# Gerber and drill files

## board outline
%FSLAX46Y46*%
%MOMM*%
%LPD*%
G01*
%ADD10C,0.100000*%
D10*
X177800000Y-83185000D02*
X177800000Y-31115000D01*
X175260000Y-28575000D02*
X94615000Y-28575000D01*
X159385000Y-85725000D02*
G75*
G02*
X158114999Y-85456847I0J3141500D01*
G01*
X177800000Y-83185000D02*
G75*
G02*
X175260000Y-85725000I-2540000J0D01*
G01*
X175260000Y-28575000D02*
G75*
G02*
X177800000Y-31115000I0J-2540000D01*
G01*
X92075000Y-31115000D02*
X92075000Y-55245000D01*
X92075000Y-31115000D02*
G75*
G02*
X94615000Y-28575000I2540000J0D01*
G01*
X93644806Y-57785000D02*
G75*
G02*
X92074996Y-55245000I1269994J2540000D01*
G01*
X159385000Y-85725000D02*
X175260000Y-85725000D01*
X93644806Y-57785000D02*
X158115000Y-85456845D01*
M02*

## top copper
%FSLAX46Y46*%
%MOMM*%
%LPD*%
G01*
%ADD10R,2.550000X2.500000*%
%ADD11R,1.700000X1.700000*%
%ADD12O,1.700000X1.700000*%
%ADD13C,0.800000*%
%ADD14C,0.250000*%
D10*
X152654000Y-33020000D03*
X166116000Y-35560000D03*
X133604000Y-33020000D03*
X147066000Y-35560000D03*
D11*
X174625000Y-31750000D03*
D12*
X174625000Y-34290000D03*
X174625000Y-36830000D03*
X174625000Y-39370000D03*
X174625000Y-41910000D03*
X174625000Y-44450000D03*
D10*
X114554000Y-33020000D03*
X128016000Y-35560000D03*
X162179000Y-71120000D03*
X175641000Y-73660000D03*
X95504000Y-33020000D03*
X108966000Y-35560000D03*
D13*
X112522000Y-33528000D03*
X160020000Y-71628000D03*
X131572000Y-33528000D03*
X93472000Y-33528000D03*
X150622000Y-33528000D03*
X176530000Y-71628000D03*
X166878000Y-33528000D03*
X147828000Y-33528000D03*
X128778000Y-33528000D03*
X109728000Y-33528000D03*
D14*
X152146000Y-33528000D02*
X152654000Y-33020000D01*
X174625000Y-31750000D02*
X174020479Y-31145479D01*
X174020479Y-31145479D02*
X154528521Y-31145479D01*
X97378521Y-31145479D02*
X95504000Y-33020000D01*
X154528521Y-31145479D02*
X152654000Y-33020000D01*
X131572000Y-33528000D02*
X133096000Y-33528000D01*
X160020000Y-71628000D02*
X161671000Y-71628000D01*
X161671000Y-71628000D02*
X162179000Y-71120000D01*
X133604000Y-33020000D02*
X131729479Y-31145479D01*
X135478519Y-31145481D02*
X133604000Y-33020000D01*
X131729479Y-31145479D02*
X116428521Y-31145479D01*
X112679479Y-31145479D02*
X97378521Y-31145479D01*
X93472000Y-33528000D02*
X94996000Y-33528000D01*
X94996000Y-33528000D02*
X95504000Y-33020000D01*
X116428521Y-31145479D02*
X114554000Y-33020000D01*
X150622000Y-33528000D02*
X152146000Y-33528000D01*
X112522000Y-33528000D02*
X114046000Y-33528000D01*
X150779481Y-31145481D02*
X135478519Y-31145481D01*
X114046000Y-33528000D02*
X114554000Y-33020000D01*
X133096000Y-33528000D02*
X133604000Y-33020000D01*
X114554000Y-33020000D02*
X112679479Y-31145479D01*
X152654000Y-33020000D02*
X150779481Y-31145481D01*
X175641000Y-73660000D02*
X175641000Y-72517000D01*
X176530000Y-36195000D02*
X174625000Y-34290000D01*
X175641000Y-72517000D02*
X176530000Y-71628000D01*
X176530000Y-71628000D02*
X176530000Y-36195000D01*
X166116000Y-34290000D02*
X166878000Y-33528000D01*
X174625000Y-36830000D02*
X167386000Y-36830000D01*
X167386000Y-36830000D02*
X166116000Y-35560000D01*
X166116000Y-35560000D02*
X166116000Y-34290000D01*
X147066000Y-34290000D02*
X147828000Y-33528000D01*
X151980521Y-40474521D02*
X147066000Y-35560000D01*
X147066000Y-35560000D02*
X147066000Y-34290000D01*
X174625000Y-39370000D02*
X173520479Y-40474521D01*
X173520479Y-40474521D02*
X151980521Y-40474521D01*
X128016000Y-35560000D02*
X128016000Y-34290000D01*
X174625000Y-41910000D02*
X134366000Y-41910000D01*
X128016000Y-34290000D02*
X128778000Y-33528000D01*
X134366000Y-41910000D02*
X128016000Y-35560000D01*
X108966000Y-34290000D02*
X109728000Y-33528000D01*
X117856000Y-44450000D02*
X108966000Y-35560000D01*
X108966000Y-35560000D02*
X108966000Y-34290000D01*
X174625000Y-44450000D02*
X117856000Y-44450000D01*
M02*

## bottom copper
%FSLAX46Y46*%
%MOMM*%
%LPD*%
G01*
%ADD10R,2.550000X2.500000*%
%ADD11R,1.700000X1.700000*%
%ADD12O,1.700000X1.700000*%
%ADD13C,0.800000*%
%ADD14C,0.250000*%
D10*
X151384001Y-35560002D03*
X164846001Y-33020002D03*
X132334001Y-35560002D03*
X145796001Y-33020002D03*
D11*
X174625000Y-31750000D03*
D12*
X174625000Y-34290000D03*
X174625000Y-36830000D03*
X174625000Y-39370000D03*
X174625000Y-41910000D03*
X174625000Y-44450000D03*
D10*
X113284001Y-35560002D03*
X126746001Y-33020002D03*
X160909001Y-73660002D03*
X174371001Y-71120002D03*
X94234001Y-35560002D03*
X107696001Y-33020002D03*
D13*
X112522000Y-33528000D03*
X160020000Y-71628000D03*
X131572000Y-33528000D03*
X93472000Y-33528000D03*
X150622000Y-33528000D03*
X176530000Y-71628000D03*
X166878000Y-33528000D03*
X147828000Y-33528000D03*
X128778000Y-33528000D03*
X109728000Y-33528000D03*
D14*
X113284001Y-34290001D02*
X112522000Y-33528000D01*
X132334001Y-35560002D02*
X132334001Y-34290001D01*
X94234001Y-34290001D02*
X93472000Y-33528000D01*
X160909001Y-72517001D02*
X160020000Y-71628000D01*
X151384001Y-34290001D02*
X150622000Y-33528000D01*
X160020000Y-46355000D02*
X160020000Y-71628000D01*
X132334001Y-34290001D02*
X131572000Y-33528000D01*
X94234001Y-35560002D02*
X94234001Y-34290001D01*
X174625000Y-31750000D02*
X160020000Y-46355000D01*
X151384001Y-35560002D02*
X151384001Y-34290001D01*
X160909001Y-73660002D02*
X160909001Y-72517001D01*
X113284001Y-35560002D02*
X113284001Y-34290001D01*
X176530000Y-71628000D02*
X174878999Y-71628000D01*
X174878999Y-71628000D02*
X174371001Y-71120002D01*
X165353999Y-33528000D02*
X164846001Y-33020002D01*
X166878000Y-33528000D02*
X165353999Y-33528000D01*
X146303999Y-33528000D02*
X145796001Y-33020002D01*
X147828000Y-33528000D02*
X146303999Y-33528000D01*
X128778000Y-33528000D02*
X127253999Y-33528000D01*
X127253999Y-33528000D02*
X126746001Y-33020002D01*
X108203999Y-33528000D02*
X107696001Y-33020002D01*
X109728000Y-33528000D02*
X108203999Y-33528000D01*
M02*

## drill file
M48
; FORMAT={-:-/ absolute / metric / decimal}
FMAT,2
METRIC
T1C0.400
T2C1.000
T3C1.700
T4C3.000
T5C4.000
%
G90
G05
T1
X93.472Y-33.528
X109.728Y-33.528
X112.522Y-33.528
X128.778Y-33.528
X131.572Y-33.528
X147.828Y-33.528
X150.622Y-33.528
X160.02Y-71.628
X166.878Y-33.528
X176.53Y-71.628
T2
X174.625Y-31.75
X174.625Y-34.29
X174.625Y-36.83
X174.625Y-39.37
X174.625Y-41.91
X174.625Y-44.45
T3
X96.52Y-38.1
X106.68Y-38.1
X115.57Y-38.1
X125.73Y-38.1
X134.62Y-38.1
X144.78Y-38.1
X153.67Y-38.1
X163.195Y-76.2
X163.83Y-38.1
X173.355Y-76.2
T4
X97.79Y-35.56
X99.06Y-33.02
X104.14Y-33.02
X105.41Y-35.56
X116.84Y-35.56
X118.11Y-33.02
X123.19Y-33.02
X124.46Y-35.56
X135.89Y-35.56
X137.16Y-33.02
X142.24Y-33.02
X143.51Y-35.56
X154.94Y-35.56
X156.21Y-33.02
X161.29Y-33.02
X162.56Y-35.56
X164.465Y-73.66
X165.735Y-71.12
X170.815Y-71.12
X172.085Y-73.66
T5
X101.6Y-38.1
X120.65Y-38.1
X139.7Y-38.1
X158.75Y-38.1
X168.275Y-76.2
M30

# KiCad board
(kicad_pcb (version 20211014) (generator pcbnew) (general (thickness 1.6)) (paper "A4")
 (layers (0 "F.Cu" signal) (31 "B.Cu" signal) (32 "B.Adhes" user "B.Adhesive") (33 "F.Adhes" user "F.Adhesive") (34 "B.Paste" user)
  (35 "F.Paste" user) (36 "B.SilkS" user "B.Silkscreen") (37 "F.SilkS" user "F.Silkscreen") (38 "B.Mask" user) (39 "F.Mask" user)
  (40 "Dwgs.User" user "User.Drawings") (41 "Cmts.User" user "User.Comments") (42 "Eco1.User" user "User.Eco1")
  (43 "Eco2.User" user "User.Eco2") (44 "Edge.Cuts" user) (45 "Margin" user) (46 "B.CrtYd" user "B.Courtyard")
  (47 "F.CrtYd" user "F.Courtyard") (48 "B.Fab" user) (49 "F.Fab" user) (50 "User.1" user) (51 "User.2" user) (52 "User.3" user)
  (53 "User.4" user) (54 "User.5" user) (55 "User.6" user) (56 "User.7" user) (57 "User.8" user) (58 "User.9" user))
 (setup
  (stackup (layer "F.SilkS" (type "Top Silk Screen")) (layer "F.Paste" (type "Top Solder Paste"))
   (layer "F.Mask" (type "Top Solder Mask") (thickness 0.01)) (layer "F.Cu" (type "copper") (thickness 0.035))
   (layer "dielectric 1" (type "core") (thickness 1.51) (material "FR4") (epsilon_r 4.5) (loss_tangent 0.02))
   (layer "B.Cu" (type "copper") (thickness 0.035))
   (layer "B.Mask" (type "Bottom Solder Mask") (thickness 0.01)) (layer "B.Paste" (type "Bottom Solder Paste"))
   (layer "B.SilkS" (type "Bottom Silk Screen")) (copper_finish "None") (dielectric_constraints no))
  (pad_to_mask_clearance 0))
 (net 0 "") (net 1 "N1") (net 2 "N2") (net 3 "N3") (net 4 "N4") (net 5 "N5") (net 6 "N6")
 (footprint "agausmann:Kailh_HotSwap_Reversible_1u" (layer "F.Cu") (at 158.75 38.1)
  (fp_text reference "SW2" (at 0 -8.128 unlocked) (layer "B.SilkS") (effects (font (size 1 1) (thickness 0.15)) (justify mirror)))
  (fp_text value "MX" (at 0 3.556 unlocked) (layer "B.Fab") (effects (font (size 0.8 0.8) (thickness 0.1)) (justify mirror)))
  (pad "" np_thru_hole circle (at -2.54 -5.08) (size 3 3) (drill 3) (layers F&B.Cu *.Mask))
  (pad "" np_thru_hole circle (at 5.08 0) (size 1.7 1.7) (drill 1.7) (layers *.Cu *.Mask))
  (pad "" np_thru_hole circle (at 0 0) (size 4 4) (drill 4) (layers *.Cu *.Mask))
  (pad "" np_thru_hole circle (at -5.08 0) (size 1.7 1.7) (drill 1.7) (layers *.Cu *.Mask))
  (pad "" np_thru_hole circle (at 3.81 -2.54) (size 3 3) (drill 3) (layers F&B.Cu *.Mask))
  (pad "" np_thru_hole circle (at 2.540001 -5.079998) (size 3 3) (drill 3) (layers F&B.Cu *.Mask))
  (pad "" np_thru_hole circle (at -3.809999 -2.539998) (size 3 3) (drill 3) (layers F&B.Cu *.Mask))
  (pad "1" smd rect (at -7.365999 -2.539998) (size 2.55 2.5) (layers "B.Cu" "B.Paste" "B.Mask") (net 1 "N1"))
  (pad "1" smd rect (at -6.096 -5.08) (size 2.55 2.5) (layers "F.Cu" "F.Paste" "F.Mask") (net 1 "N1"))
  (pad "2" smd rect (at 6.096001 -5.079998) (size 2.55 2.5) (layers "B.Cu" "B.Paste" "B.Mask") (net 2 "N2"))
  (pad "2" smd rect (at 7.366 -2.54) (size 2.55 2.5) (layers "F.Cu" "F.Paste" "F.Mask") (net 2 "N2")))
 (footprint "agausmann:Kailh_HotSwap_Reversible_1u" (layer "F.Cu") (at 139.7 38.1)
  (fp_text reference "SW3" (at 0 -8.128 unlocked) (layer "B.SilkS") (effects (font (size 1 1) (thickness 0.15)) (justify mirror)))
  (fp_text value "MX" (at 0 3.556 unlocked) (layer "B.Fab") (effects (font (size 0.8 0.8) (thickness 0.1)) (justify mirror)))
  (pad "" np_thru_hole circle (at 3.81 -2.54) (size 3 3) (drill 3) (layers F&B.Cu *.Mask))
  (pad "" np_thru_hole circle (at -5.08 0) (size 1.7 1.7) (drill 1.7) (layers *.Cu *.Mask))
  (pad "" np_thru_hole circle (at -3.809999 -2.539998) (size 3 3) (drill 3) (layers F&B.Cu *.Mask))
  (pad "" np_thru_hole circle (at 0 0) (size 4 4) (drill 4) (layers *.Cu *.Mask))
  (pad "" np_thru_hole circle (at 5.08 0) (size 1.7 1.7) (drill 1.7) (layers *.Cu *.Mask))
  (pad "" np_thru_hole circle (at 2.540001 -5.079998) (size 3 3) (drill 3) (layers F&B.Cu *.Mask))
  (pad "" np_thru_hole circle (at -2.54 -5.08) (size 3 3) (drill 3) (layers F&B.Cu *.Mask))
  (pad "1" smd rect (at -7.365999 -2.539998) (size 2.55 2.5) (layers "B.Cu" "B.Paste" "B.Mask") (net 1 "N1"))
  (pad "1" smd rect (at -6.096 -5.08) (size 2.55 2.5) (layers "F.Cu" "F.Paste" "F.Mask") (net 1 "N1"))
  (pad "2" smd rect (at 7.366 -2.54) (size 2.55 2.5) (layers "F.Cu" "F.Paste" "F.Mask") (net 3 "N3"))
  (pad "2" smd rect (at 6.096001 -5.079998) (size 2.55 2.5) (layers "B.Cu" "B.Paste" "B.Mask") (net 3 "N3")))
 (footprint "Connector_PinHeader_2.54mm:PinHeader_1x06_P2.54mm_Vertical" (layer "F.Cu") (at 174.625 31.75)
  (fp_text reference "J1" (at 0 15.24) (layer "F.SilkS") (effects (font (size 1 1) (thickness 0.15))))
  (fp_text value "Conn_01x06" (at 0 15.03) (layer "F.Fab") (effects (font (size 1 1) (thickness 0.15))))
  (pad "1" thru_hole rect (at 0 0) (size 1.7 1.7) (drill 1) (layers *.Cu *.Mask) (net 1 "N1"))
  (pad "2" thru_hole oval (at 0 2.54) (size 1.7 1.7) (drill 1) (layers *.Cu *.Mask) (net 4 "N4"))
  (pad "3" thru_hole oval (at 0 5.08) (size 1.7 1.7) (drill 1) (layers *.Cu *.Mask) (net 2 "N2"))
  (pad "4" thru_hole oval (at 0 7.62) (size 1.7 1.7) (drill 1) (layers *.Cu *.Mask) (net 3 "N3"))
  (pad "5" thru_hole oval (at 0 10.16) (size 1.7 1.7) (drill 1) (layers *.Cu *.Mask) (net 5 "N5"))
  (pad "6" thru_hole oval (at 0 12.7) (size 1.7 1.7) (drill 1) (layers *.Cu *.Mask) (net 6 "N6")))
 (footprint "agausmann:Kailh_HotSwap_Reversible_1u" (layer "F.Cu") (at 120.65 38.1)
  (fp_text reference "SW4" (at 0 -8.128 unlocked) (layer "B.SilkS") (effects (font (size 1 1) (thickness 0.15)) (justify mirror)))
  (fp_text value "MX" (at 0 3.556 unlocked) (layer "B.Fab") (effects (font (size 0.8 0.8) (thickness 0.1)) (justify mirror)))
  (pad "" np_thru_hole circle (at 0 0) (size 4 4) (drill 4) (layers *.Cu *.Mask))
  (pad "" np_thru_hole circle (at 2.540001 -5.079998) (size 3 3) (drill 3) (layers F&B.Cu *.Mask))
  (pad "" np_thru_hole circle (at 3.81 -2.54) (size 3 3) (drill 3) (layers F&B.Cu *.Mask))
  (pad "" np_thru_hole circle (at -2.54 -5.08) (size 3 3) (drill 3) (layers F&B.Cu *.Mask))
  (pad "" np_thru_hole circle (at -3.809999 -2.539998) (size 3 3) (drill 3) (layers F&B.Cu *.Mask))
  (pad "" np_thru_hole circle (at 5.08 0) (size 1.7 1.7) (drill 1.7) (layers *.Cu *.Mask))
  (pad "" np_thru_hole circle (at -5.08 0) (size 1.7 1.7) (drill 1.7) (layers *.Cu *.Mask))
  (pad "1" smd rect (at -7.365999 -2.539998) (size 2.55 2.5) (layers "B.Cu" "B.Paste" "B.Mask") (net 1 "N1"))
  (pad "1" smd rect (at -6.096 -5.08) (size 2.55 2.5) (layers "F.Cu" "F.Paste" "F.Mask") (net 1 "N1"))
  (pad "2" smd rect (at 6.096001 -5.079998) (size 2.55 2.5) (layers "B.Cu" "B.Paste" "B.Mask") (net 5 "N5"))
  (pad "2" smd rect (at 7.366 -2.54) (size 2.55 2.5) (layers "F.Cu" "F.Paste" "F.Mask") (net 5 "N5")))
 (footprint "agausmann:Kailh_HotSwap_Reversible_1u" (layer "F.Cu") (at 168.275 76.2)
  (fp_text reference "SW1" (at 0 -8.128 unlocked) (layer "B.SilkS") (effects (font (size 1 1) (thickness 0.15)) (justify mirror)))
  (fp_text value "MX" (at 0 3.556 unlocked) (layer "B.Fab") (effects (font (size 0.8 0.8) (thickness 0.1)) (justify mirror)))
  (pad "" np_thru_hole circle (at 3.81 -2.54) (size 3 3) (drill 3) (layers F&B.Cu *.Mask))
  (pad "" np_thru_hole circle (at -5.08 0) (size 1.7 1.7) (drill 1.7) (layers *.Cu *.Mask))
  (pad "" np_thru_hole circle (at -3.809999 -2.539998) (size 3 3) (drill 3) (layers F&B.Cu *.Mask))
  (pad "" np_thru_hole circle (at 2.540001 -5.079998) (size 3 3) (drill 3) (layers F&B.Cu *.Mask))
  (pad "" np_thru_hole circle (at 0 0) (size 4 4) (drill 4) (layers *.Cu *.Mask))
  (pad "" np_thru_hole circle (at 5.08 0) (size 1.7 1.7) (drill 1.7) (layers *.Cu *.Mask))
  (pad "" np_thru_hole circle (at -2.54 -5.08) (size 3 3) (drill 3) (layers F&B.Cu *.Mask))
  (pad "1" smd rect (at -6.096 -5.08) (size 2.55 2.5) (layers "F.Cu" "F.Paste" "F.Mask") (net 1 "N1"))
  (pad "1" smd rect (at -7.365999 -2.539998) (size 2.55 2.5) (layers "B.Cu" "B.Paste" "B.Mask") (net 1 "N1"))
  (pad "2" smd rect (at 6.096001 -5.079998) (size 2.55 2.5) (layers "B.Cu" "B.Paste" "B.Mask") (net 4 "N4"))
  (pad "2" smd rect (at 7.366 -2.54) (size 2.55 2.5) (layers "F.Cu" "F.Paste" "F.Mask") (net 4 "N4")))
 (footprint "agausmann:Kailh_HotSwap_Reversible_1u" (layer "F.Cu") (at 101.6 38.1)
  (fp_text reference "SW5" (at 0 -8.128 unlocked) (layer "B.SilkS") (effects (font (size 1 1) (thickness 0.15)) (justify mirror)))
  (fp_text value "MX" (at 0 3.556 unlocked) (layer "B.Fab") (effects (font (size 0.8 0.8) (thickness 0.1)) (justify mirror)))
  (pad "" np_thru_hole circle (at 3.81 -2.54) (size 3 3) (drill 3) (layers F&B.Cu *.Mask))
  (pad "" np_thru_hole circle (at 2.540001 -5.079998) (size 3 3) (drill 3) (layers F&B.Cu *.Mask))
  (pad "" np_thru_hole circle (at 5.08 0) (size 1.7 1.7) (drill 1.7) (layers *.Cu *.Mask))
  (pad "" np_thru_hole circle (at -5.08 0) (size 1.7 1.7) (drill 1.7) (layers *.Cu *.Mask))
  (pad "" np_thru_hole circle (at 0 0) (size 4 4) (drill 4) (layers *.Cu *.Mask))
  (pad "" np_thru_hole circle (at -2.54 -5.08) (size 3 3) (drill 3) (layers F&B.Cu *.Mask))
  (pad "" np_thru_hole circle (at -3.809999 -2.539998) (size 3 3) (drill 3) (layers F&B.Cu *.Mask))
  (pad "1" smd rect (at -6.096 -5.08) (size 2.55 2.5) (layers "F.Cu" "F.Paste" "F.Mask") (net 1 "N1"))
  (pad "1" smd rect (at -7.365999 -2.539998) (size 2.55 2.5) (layers "B.Cu" "B.Paste" "B.Mask") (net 1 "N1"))
  (pad "2" smd rect (at 6.096001 -5.079998) (size 2.55 2.5) (layers "B.Cu" "B.Paste" "B.Mask") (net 6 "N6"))
  (pad "2" smd rect (at 7.366 -2.54) (size 2.55 2.5) (layers "F.Cu" "F.Paste" "F.Mask") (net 6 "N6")))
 (gr_line (start 177.8 83.185) (end 177.8 31.115) (layer "Edge.Cuts") (width 0.1))
 (gr_line (start 175.26 28.575) (end 94.615 28.575) (layer "Edge.Cuts") (width 0.1))
 (gr_arc (start 159.385 85.725) (mid 158.735999 85.65723) (end 158.115 85.456845) (layer "Edge.Cuts") (width 0.1))
 (gr_arc (start 177.8 83.185) (mid 177.056051 84.981051) (end 175.26 85.725) (layer "Edge.Cuts") (width 0.1))
 (gr_arc (start 175.26 28.575) (mid 177.056051 29.318949) (end 177.8 31.115) (layer "Edge.Cuts") (width 0.1))
 (gr_line (start 92.075 31.115) (end 92.075 55.245) (layer "Edge.Cuts") (width 0.1))
 (gr_arc (start 92.075 31.115) (mid 92.818949 29.318949) (end 94.615 28.575) (layer "Edge.Cuts") (width 0.1))
 (gr_arc (start 93.644806 57.785) (mid 92.499122 56.737975) (end 92.075 55.245) (layer "Edge.Cuts") (width 0.1))
 (gr_line (start 159.385 85.725) (end 175.26 85.725) (layer "Edge.Cuts") (width 0.1))
 (gr_line (start 93.644806 57.785) (end 158.115 85.456845) (layer "Edge.Cuts") (width 0.1))
 (segment (start 152.146 33.528) (end 152.654 33.02) (width 0.25) (layer "F.Cu") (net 1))
 (segment (start 174.625 31.75) (end 174.020479 31.145479) (width 0.25) (layer "F.Cu") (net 1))
 (segment (start 174.020479 31.145479) (end 154.528521 31.145479) (width 0.25) (layer "F.Cu") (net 1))
 (segment (start 97.378521 31.145479) (end 95.504 33.02) (width 0.25) (layer "F.Cu") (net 1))
 (segment (start 154.528521 31.145479) (end 152.654 33.02) (width 0.25) (layer "F.Cu") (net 1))
 (segment (start 131.572 33.528) (end 133.096 33.528) (width 0.25) (layer "F.Cu") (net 1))
 (segment (start 160.02 71.628) (end 161.671 71.628) (width 0.25) (layer "F.Cu") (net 1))
 (segment (start 161.671 71.628) (end 162.179 71.12) (width 0.25) (layer "F.Cu") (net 1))
 (segment (start 133.604 33.02) (end 131.729479 31.145479) (width 0.25) (layer "F.Cu") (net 1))
 (segment (start 135.478519 31.145481) (end 133.604 33.02) (width 0.25) (layer "F.Cu") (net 1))
 (segment (start 131.729479 31.145479) (end 116.428521 31.145479) (width 0.25) (layer "F.Cu") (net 1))
 (segment (start 112.679479 31.145479) (end 97.378521 31.145479) (width 0.25) (layer "F.Cu") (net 1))
 (segment (start 93.472 33.528) (end 94.996 33.528) (width 0.25) (layer "F.Cu") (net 1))
 (segment (start 94.996 33.528) (end 95.504 33.02) (width 0.25) (layer "F.Cu") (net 1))
 (segment (start 116.428521 31.145479) (end 114.554 33.02) (width 0.25) (layer "F.Cu") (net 1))
 (segment (start 150.622 33.528) (end 152.146 33.528) (width 0.25) (layer "F.Cu") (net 1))
 (segment (start 112.522 33.528) (end 114.046 33.528) (width 0.25) (layer "F.Cu") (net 1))
 (segment (start 150.779481 31.145481) (end 135.478519 31.145481) (width 0.25) (layer "F.Cu") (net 1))
 (segment (start 114.046 33.528) (end 114.554 33.02) (width 0.25) (layer "F.Cu") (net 1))
 (segment (start 133.096 33.528) (end 133.604 33.02) (width 0.25) (layer "F.Cu") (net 1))
 (segment (start 114.554 33.02) (end 112.679479 31.145479) (width 0.25) (layer "F.Cu") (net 1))
 (segment (start 152.654 33.02) (end 150.779481 31.145481) (width 0.25) (layer "F.Cu") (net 1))
 (via (at 112.522 33.528) (size 0.8) (drill 0.4) (layers "F.Cu" "B.Cu") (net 1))
 (via (at 160.02 71.628) (size 0.8) (drill 0.4) (layers "F.Cu" "B.Cu") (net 1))
 (via (at 131.572 33.528) (size 0.8) (drill 0.4) (layers "F.Cu" "B.Cu") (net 1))
 (via (at 93.472 33.528) (size 0.8) (drill 0.4) (layers "F.Cu" "B.Cu") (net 1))
 (via (at 150.622 33.528) (size 0.8) (drill 0.4) (layers "F.Cu" "B.Cu") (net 1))
 (segment (start 113.284001 34.290001) (end 112.522 33.528) (width 0.25) (layer "B.Cu") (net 1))
 (segment (start 132.334001 35.560002) (end 132.334001 34.290001) (width 0.25) (layer "B.Cu") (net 1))
 (segment (start 94.234001 34.290001) (end 93.472 33.528) (width 0.25) (layer "B.Cu") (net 1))
 (segment (start 160.909001 72.517001) (end 160.02 71.628) (width 0.25) (layer "B.Cu") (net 1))
 (segment (start 151.384001 34.290001) (end 150.622 33.528) (width 0.25) (layer "B.Cu") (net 1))
 (segment (start 160.02 46.355) (end 160.02 71.628) (width 0.25) (layer "B.Cu") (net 1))
 (segment (start 132.334001 34.290001) (end 131.572 33.528) (width 0.25) (layer "B.Cu") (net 1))
 (segment (start 94.234001 35.560002) (end 94.234001 34.290001) (width 0.25) (layer "B.Cu") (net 1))
 (segment (start 174.625 31.75) (end 160.02 46.355) (width 0.25) (layer "B.Cu") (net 1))
 (segment (start 151.384001 35.560002) (end 151.384001 34.290001) (width 0.25) (layer "B.Cu") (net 1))
 (segment (start 160.909001 73.660002) (end 160.909001 72.517001) (width 0.25) (layer "B.Cu") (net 1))
 (segment (start 113.284001 35.560002) (end 113.284001 34.290001) (width 0.25) (layer "B.Cu") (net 1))
 (segment (start 175.641 73.66) (end 175.641 72.517) (width 0.25) (layer "F.Cu") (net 4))
 (segment (start 176.53 36.195) (end 174.625 34.29) (width 0.25) (layer "F.Cu") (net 4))
 (segment (start 175.641 72.517) (end 176.53 71.628) (width 0.25) (layer "F.Cu") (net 4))
 (segment (start 176.53 71.628) (end 176.53 36.195) (width 0.25) (layer "F.Cu") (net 4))
 (via (at 176.53 71.628) (size 0.8) (drill 0.4) (layers "F.Cu" "B.Cu") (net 4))
 (segment (start 176.53 71.628) (end 174.878999 71.628) (width 0.25) (layer "B.Cu") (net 4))
 (segment (start 174.878999 71.628) (end 174.371001 71.120002) (width 0.25) (layer "B.Cu") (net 4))
 (segment (start 166.116 34.29) (end 166.878 33.528) (width 0.25) (layer "F.Cu") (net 2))
 (segment (start 174.625 36.83) (end 167.386 36.83) (width 0.25) (layer "F.Cu") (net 2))
 (segment (start 167.386 36.83) (end 166.116 35.56) (width 0.25) (layer "F.Cu") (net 2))
 (segment (start 166.116 35.56) (end 166.116 34.29) (width 0.25) (layer "F.Cu") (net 2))
 (via (at 166.878 33.528) (size 0.8) (drill 0.4) (layers "F.Cu" "B.Cu") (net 2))
 (segment (start 165.353999 33.528) (end 164.846001 33.020002) (width 0.25) (layer "B.Cu") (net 2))
 (segment (start 166.878 33.528) (end 165.353999 33.528) (width 0.25) (layer "B.Cu") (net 2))
 (segment (start 147.066 34.29) (end 147.828 33.528) (width 0.25) (layer "F.Cu") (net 3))
 (segment (start 151.980521 40.474521) (end 147.066 35.56) (width 0.25) (layer "F.Cu") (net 3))
 (segment (start 147.066 35.56) (end 147.066 34.29) (width 0.25) (layer "F.Cu") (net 3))
 (segment (start 174.625 39.37) (end 173.520479 40.474521) (width 0.25) (layer "F.Cu") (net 3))
 (segment (start 173.520479 40.474521) (end 151.980521 40.474521) (width 0.25) (layer "F.Cu") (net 3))
 (via (at 147.828 33.528) (size 0.8) (drill 0.4) (layers "F.Cu" "B.Cu") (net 3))
 (segment (start 146.303999 33.528) (end 145.796001 33.020002) (width 0.25) (layer "B.Cu") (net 3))
 (segment (start 147.828 33.528) (end 146.303999 33.528) (width 0.25) (layer "B.Cu") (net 3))
 (segment (start 128.016 35.56) (end 128.016 34.29) (width 0.25) (layer "F.Cu") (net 5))
 (segment (start 174.625 41.91) (end 134.366 41.91) (width 0.25) (layer "F.Cu") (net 5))
 (segment (start 128.016 34.29) (end 128.778 33.528) (width 0.25) (layer "F.Cu") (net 5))
 (segment (start 134.366 41.91) (end 128.016 35.56) (width 0.25) (layer "F.Cu") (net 5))
 (via (at 128.778 33.528) (size 0.8) (drill 0.4) (layers "F.Cu" "B.Cu") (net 5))
 (segment (start 128.778 33.528) (end 127.253999 33.528) (width 0.25) (layer "B.Cu") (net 5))
 (segment (start 127.253999 33.528) (end 126.746001 33.020002) (width 0.25) (layer "B.Cu") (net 5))
 (segment (start 108.966 34.29) (end 109.728 33.528) (width 0.25) (layer "F.Cu") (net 6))
 (segment (start 117.856 44.45) (end 108.966 35.56) (width 0.25) (layer "F.Cu") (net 6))
 (segment (start 108.966 35.56) (end 108.966 34.29) (width 0.25) (layer "F.Cu") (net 6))
 (segment (start 174.625 44.45) (end 117.856 44.45) (width 0.25) (layer "F.Cu") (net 6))
 (via (at 109.728 33.528) (size 0.8) (drill 0.4) (layers "F.Cu" "B.Cu") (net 6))
 (segment (start 108.203999 33.528) (end 107.696001 33.020002) (width 0.25) (layer "B.Cu") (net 6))
 (segment (start 109.728 33.528) (end 108.203999 33.528) (width 0.25) (layer "B.Cu") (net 6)))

